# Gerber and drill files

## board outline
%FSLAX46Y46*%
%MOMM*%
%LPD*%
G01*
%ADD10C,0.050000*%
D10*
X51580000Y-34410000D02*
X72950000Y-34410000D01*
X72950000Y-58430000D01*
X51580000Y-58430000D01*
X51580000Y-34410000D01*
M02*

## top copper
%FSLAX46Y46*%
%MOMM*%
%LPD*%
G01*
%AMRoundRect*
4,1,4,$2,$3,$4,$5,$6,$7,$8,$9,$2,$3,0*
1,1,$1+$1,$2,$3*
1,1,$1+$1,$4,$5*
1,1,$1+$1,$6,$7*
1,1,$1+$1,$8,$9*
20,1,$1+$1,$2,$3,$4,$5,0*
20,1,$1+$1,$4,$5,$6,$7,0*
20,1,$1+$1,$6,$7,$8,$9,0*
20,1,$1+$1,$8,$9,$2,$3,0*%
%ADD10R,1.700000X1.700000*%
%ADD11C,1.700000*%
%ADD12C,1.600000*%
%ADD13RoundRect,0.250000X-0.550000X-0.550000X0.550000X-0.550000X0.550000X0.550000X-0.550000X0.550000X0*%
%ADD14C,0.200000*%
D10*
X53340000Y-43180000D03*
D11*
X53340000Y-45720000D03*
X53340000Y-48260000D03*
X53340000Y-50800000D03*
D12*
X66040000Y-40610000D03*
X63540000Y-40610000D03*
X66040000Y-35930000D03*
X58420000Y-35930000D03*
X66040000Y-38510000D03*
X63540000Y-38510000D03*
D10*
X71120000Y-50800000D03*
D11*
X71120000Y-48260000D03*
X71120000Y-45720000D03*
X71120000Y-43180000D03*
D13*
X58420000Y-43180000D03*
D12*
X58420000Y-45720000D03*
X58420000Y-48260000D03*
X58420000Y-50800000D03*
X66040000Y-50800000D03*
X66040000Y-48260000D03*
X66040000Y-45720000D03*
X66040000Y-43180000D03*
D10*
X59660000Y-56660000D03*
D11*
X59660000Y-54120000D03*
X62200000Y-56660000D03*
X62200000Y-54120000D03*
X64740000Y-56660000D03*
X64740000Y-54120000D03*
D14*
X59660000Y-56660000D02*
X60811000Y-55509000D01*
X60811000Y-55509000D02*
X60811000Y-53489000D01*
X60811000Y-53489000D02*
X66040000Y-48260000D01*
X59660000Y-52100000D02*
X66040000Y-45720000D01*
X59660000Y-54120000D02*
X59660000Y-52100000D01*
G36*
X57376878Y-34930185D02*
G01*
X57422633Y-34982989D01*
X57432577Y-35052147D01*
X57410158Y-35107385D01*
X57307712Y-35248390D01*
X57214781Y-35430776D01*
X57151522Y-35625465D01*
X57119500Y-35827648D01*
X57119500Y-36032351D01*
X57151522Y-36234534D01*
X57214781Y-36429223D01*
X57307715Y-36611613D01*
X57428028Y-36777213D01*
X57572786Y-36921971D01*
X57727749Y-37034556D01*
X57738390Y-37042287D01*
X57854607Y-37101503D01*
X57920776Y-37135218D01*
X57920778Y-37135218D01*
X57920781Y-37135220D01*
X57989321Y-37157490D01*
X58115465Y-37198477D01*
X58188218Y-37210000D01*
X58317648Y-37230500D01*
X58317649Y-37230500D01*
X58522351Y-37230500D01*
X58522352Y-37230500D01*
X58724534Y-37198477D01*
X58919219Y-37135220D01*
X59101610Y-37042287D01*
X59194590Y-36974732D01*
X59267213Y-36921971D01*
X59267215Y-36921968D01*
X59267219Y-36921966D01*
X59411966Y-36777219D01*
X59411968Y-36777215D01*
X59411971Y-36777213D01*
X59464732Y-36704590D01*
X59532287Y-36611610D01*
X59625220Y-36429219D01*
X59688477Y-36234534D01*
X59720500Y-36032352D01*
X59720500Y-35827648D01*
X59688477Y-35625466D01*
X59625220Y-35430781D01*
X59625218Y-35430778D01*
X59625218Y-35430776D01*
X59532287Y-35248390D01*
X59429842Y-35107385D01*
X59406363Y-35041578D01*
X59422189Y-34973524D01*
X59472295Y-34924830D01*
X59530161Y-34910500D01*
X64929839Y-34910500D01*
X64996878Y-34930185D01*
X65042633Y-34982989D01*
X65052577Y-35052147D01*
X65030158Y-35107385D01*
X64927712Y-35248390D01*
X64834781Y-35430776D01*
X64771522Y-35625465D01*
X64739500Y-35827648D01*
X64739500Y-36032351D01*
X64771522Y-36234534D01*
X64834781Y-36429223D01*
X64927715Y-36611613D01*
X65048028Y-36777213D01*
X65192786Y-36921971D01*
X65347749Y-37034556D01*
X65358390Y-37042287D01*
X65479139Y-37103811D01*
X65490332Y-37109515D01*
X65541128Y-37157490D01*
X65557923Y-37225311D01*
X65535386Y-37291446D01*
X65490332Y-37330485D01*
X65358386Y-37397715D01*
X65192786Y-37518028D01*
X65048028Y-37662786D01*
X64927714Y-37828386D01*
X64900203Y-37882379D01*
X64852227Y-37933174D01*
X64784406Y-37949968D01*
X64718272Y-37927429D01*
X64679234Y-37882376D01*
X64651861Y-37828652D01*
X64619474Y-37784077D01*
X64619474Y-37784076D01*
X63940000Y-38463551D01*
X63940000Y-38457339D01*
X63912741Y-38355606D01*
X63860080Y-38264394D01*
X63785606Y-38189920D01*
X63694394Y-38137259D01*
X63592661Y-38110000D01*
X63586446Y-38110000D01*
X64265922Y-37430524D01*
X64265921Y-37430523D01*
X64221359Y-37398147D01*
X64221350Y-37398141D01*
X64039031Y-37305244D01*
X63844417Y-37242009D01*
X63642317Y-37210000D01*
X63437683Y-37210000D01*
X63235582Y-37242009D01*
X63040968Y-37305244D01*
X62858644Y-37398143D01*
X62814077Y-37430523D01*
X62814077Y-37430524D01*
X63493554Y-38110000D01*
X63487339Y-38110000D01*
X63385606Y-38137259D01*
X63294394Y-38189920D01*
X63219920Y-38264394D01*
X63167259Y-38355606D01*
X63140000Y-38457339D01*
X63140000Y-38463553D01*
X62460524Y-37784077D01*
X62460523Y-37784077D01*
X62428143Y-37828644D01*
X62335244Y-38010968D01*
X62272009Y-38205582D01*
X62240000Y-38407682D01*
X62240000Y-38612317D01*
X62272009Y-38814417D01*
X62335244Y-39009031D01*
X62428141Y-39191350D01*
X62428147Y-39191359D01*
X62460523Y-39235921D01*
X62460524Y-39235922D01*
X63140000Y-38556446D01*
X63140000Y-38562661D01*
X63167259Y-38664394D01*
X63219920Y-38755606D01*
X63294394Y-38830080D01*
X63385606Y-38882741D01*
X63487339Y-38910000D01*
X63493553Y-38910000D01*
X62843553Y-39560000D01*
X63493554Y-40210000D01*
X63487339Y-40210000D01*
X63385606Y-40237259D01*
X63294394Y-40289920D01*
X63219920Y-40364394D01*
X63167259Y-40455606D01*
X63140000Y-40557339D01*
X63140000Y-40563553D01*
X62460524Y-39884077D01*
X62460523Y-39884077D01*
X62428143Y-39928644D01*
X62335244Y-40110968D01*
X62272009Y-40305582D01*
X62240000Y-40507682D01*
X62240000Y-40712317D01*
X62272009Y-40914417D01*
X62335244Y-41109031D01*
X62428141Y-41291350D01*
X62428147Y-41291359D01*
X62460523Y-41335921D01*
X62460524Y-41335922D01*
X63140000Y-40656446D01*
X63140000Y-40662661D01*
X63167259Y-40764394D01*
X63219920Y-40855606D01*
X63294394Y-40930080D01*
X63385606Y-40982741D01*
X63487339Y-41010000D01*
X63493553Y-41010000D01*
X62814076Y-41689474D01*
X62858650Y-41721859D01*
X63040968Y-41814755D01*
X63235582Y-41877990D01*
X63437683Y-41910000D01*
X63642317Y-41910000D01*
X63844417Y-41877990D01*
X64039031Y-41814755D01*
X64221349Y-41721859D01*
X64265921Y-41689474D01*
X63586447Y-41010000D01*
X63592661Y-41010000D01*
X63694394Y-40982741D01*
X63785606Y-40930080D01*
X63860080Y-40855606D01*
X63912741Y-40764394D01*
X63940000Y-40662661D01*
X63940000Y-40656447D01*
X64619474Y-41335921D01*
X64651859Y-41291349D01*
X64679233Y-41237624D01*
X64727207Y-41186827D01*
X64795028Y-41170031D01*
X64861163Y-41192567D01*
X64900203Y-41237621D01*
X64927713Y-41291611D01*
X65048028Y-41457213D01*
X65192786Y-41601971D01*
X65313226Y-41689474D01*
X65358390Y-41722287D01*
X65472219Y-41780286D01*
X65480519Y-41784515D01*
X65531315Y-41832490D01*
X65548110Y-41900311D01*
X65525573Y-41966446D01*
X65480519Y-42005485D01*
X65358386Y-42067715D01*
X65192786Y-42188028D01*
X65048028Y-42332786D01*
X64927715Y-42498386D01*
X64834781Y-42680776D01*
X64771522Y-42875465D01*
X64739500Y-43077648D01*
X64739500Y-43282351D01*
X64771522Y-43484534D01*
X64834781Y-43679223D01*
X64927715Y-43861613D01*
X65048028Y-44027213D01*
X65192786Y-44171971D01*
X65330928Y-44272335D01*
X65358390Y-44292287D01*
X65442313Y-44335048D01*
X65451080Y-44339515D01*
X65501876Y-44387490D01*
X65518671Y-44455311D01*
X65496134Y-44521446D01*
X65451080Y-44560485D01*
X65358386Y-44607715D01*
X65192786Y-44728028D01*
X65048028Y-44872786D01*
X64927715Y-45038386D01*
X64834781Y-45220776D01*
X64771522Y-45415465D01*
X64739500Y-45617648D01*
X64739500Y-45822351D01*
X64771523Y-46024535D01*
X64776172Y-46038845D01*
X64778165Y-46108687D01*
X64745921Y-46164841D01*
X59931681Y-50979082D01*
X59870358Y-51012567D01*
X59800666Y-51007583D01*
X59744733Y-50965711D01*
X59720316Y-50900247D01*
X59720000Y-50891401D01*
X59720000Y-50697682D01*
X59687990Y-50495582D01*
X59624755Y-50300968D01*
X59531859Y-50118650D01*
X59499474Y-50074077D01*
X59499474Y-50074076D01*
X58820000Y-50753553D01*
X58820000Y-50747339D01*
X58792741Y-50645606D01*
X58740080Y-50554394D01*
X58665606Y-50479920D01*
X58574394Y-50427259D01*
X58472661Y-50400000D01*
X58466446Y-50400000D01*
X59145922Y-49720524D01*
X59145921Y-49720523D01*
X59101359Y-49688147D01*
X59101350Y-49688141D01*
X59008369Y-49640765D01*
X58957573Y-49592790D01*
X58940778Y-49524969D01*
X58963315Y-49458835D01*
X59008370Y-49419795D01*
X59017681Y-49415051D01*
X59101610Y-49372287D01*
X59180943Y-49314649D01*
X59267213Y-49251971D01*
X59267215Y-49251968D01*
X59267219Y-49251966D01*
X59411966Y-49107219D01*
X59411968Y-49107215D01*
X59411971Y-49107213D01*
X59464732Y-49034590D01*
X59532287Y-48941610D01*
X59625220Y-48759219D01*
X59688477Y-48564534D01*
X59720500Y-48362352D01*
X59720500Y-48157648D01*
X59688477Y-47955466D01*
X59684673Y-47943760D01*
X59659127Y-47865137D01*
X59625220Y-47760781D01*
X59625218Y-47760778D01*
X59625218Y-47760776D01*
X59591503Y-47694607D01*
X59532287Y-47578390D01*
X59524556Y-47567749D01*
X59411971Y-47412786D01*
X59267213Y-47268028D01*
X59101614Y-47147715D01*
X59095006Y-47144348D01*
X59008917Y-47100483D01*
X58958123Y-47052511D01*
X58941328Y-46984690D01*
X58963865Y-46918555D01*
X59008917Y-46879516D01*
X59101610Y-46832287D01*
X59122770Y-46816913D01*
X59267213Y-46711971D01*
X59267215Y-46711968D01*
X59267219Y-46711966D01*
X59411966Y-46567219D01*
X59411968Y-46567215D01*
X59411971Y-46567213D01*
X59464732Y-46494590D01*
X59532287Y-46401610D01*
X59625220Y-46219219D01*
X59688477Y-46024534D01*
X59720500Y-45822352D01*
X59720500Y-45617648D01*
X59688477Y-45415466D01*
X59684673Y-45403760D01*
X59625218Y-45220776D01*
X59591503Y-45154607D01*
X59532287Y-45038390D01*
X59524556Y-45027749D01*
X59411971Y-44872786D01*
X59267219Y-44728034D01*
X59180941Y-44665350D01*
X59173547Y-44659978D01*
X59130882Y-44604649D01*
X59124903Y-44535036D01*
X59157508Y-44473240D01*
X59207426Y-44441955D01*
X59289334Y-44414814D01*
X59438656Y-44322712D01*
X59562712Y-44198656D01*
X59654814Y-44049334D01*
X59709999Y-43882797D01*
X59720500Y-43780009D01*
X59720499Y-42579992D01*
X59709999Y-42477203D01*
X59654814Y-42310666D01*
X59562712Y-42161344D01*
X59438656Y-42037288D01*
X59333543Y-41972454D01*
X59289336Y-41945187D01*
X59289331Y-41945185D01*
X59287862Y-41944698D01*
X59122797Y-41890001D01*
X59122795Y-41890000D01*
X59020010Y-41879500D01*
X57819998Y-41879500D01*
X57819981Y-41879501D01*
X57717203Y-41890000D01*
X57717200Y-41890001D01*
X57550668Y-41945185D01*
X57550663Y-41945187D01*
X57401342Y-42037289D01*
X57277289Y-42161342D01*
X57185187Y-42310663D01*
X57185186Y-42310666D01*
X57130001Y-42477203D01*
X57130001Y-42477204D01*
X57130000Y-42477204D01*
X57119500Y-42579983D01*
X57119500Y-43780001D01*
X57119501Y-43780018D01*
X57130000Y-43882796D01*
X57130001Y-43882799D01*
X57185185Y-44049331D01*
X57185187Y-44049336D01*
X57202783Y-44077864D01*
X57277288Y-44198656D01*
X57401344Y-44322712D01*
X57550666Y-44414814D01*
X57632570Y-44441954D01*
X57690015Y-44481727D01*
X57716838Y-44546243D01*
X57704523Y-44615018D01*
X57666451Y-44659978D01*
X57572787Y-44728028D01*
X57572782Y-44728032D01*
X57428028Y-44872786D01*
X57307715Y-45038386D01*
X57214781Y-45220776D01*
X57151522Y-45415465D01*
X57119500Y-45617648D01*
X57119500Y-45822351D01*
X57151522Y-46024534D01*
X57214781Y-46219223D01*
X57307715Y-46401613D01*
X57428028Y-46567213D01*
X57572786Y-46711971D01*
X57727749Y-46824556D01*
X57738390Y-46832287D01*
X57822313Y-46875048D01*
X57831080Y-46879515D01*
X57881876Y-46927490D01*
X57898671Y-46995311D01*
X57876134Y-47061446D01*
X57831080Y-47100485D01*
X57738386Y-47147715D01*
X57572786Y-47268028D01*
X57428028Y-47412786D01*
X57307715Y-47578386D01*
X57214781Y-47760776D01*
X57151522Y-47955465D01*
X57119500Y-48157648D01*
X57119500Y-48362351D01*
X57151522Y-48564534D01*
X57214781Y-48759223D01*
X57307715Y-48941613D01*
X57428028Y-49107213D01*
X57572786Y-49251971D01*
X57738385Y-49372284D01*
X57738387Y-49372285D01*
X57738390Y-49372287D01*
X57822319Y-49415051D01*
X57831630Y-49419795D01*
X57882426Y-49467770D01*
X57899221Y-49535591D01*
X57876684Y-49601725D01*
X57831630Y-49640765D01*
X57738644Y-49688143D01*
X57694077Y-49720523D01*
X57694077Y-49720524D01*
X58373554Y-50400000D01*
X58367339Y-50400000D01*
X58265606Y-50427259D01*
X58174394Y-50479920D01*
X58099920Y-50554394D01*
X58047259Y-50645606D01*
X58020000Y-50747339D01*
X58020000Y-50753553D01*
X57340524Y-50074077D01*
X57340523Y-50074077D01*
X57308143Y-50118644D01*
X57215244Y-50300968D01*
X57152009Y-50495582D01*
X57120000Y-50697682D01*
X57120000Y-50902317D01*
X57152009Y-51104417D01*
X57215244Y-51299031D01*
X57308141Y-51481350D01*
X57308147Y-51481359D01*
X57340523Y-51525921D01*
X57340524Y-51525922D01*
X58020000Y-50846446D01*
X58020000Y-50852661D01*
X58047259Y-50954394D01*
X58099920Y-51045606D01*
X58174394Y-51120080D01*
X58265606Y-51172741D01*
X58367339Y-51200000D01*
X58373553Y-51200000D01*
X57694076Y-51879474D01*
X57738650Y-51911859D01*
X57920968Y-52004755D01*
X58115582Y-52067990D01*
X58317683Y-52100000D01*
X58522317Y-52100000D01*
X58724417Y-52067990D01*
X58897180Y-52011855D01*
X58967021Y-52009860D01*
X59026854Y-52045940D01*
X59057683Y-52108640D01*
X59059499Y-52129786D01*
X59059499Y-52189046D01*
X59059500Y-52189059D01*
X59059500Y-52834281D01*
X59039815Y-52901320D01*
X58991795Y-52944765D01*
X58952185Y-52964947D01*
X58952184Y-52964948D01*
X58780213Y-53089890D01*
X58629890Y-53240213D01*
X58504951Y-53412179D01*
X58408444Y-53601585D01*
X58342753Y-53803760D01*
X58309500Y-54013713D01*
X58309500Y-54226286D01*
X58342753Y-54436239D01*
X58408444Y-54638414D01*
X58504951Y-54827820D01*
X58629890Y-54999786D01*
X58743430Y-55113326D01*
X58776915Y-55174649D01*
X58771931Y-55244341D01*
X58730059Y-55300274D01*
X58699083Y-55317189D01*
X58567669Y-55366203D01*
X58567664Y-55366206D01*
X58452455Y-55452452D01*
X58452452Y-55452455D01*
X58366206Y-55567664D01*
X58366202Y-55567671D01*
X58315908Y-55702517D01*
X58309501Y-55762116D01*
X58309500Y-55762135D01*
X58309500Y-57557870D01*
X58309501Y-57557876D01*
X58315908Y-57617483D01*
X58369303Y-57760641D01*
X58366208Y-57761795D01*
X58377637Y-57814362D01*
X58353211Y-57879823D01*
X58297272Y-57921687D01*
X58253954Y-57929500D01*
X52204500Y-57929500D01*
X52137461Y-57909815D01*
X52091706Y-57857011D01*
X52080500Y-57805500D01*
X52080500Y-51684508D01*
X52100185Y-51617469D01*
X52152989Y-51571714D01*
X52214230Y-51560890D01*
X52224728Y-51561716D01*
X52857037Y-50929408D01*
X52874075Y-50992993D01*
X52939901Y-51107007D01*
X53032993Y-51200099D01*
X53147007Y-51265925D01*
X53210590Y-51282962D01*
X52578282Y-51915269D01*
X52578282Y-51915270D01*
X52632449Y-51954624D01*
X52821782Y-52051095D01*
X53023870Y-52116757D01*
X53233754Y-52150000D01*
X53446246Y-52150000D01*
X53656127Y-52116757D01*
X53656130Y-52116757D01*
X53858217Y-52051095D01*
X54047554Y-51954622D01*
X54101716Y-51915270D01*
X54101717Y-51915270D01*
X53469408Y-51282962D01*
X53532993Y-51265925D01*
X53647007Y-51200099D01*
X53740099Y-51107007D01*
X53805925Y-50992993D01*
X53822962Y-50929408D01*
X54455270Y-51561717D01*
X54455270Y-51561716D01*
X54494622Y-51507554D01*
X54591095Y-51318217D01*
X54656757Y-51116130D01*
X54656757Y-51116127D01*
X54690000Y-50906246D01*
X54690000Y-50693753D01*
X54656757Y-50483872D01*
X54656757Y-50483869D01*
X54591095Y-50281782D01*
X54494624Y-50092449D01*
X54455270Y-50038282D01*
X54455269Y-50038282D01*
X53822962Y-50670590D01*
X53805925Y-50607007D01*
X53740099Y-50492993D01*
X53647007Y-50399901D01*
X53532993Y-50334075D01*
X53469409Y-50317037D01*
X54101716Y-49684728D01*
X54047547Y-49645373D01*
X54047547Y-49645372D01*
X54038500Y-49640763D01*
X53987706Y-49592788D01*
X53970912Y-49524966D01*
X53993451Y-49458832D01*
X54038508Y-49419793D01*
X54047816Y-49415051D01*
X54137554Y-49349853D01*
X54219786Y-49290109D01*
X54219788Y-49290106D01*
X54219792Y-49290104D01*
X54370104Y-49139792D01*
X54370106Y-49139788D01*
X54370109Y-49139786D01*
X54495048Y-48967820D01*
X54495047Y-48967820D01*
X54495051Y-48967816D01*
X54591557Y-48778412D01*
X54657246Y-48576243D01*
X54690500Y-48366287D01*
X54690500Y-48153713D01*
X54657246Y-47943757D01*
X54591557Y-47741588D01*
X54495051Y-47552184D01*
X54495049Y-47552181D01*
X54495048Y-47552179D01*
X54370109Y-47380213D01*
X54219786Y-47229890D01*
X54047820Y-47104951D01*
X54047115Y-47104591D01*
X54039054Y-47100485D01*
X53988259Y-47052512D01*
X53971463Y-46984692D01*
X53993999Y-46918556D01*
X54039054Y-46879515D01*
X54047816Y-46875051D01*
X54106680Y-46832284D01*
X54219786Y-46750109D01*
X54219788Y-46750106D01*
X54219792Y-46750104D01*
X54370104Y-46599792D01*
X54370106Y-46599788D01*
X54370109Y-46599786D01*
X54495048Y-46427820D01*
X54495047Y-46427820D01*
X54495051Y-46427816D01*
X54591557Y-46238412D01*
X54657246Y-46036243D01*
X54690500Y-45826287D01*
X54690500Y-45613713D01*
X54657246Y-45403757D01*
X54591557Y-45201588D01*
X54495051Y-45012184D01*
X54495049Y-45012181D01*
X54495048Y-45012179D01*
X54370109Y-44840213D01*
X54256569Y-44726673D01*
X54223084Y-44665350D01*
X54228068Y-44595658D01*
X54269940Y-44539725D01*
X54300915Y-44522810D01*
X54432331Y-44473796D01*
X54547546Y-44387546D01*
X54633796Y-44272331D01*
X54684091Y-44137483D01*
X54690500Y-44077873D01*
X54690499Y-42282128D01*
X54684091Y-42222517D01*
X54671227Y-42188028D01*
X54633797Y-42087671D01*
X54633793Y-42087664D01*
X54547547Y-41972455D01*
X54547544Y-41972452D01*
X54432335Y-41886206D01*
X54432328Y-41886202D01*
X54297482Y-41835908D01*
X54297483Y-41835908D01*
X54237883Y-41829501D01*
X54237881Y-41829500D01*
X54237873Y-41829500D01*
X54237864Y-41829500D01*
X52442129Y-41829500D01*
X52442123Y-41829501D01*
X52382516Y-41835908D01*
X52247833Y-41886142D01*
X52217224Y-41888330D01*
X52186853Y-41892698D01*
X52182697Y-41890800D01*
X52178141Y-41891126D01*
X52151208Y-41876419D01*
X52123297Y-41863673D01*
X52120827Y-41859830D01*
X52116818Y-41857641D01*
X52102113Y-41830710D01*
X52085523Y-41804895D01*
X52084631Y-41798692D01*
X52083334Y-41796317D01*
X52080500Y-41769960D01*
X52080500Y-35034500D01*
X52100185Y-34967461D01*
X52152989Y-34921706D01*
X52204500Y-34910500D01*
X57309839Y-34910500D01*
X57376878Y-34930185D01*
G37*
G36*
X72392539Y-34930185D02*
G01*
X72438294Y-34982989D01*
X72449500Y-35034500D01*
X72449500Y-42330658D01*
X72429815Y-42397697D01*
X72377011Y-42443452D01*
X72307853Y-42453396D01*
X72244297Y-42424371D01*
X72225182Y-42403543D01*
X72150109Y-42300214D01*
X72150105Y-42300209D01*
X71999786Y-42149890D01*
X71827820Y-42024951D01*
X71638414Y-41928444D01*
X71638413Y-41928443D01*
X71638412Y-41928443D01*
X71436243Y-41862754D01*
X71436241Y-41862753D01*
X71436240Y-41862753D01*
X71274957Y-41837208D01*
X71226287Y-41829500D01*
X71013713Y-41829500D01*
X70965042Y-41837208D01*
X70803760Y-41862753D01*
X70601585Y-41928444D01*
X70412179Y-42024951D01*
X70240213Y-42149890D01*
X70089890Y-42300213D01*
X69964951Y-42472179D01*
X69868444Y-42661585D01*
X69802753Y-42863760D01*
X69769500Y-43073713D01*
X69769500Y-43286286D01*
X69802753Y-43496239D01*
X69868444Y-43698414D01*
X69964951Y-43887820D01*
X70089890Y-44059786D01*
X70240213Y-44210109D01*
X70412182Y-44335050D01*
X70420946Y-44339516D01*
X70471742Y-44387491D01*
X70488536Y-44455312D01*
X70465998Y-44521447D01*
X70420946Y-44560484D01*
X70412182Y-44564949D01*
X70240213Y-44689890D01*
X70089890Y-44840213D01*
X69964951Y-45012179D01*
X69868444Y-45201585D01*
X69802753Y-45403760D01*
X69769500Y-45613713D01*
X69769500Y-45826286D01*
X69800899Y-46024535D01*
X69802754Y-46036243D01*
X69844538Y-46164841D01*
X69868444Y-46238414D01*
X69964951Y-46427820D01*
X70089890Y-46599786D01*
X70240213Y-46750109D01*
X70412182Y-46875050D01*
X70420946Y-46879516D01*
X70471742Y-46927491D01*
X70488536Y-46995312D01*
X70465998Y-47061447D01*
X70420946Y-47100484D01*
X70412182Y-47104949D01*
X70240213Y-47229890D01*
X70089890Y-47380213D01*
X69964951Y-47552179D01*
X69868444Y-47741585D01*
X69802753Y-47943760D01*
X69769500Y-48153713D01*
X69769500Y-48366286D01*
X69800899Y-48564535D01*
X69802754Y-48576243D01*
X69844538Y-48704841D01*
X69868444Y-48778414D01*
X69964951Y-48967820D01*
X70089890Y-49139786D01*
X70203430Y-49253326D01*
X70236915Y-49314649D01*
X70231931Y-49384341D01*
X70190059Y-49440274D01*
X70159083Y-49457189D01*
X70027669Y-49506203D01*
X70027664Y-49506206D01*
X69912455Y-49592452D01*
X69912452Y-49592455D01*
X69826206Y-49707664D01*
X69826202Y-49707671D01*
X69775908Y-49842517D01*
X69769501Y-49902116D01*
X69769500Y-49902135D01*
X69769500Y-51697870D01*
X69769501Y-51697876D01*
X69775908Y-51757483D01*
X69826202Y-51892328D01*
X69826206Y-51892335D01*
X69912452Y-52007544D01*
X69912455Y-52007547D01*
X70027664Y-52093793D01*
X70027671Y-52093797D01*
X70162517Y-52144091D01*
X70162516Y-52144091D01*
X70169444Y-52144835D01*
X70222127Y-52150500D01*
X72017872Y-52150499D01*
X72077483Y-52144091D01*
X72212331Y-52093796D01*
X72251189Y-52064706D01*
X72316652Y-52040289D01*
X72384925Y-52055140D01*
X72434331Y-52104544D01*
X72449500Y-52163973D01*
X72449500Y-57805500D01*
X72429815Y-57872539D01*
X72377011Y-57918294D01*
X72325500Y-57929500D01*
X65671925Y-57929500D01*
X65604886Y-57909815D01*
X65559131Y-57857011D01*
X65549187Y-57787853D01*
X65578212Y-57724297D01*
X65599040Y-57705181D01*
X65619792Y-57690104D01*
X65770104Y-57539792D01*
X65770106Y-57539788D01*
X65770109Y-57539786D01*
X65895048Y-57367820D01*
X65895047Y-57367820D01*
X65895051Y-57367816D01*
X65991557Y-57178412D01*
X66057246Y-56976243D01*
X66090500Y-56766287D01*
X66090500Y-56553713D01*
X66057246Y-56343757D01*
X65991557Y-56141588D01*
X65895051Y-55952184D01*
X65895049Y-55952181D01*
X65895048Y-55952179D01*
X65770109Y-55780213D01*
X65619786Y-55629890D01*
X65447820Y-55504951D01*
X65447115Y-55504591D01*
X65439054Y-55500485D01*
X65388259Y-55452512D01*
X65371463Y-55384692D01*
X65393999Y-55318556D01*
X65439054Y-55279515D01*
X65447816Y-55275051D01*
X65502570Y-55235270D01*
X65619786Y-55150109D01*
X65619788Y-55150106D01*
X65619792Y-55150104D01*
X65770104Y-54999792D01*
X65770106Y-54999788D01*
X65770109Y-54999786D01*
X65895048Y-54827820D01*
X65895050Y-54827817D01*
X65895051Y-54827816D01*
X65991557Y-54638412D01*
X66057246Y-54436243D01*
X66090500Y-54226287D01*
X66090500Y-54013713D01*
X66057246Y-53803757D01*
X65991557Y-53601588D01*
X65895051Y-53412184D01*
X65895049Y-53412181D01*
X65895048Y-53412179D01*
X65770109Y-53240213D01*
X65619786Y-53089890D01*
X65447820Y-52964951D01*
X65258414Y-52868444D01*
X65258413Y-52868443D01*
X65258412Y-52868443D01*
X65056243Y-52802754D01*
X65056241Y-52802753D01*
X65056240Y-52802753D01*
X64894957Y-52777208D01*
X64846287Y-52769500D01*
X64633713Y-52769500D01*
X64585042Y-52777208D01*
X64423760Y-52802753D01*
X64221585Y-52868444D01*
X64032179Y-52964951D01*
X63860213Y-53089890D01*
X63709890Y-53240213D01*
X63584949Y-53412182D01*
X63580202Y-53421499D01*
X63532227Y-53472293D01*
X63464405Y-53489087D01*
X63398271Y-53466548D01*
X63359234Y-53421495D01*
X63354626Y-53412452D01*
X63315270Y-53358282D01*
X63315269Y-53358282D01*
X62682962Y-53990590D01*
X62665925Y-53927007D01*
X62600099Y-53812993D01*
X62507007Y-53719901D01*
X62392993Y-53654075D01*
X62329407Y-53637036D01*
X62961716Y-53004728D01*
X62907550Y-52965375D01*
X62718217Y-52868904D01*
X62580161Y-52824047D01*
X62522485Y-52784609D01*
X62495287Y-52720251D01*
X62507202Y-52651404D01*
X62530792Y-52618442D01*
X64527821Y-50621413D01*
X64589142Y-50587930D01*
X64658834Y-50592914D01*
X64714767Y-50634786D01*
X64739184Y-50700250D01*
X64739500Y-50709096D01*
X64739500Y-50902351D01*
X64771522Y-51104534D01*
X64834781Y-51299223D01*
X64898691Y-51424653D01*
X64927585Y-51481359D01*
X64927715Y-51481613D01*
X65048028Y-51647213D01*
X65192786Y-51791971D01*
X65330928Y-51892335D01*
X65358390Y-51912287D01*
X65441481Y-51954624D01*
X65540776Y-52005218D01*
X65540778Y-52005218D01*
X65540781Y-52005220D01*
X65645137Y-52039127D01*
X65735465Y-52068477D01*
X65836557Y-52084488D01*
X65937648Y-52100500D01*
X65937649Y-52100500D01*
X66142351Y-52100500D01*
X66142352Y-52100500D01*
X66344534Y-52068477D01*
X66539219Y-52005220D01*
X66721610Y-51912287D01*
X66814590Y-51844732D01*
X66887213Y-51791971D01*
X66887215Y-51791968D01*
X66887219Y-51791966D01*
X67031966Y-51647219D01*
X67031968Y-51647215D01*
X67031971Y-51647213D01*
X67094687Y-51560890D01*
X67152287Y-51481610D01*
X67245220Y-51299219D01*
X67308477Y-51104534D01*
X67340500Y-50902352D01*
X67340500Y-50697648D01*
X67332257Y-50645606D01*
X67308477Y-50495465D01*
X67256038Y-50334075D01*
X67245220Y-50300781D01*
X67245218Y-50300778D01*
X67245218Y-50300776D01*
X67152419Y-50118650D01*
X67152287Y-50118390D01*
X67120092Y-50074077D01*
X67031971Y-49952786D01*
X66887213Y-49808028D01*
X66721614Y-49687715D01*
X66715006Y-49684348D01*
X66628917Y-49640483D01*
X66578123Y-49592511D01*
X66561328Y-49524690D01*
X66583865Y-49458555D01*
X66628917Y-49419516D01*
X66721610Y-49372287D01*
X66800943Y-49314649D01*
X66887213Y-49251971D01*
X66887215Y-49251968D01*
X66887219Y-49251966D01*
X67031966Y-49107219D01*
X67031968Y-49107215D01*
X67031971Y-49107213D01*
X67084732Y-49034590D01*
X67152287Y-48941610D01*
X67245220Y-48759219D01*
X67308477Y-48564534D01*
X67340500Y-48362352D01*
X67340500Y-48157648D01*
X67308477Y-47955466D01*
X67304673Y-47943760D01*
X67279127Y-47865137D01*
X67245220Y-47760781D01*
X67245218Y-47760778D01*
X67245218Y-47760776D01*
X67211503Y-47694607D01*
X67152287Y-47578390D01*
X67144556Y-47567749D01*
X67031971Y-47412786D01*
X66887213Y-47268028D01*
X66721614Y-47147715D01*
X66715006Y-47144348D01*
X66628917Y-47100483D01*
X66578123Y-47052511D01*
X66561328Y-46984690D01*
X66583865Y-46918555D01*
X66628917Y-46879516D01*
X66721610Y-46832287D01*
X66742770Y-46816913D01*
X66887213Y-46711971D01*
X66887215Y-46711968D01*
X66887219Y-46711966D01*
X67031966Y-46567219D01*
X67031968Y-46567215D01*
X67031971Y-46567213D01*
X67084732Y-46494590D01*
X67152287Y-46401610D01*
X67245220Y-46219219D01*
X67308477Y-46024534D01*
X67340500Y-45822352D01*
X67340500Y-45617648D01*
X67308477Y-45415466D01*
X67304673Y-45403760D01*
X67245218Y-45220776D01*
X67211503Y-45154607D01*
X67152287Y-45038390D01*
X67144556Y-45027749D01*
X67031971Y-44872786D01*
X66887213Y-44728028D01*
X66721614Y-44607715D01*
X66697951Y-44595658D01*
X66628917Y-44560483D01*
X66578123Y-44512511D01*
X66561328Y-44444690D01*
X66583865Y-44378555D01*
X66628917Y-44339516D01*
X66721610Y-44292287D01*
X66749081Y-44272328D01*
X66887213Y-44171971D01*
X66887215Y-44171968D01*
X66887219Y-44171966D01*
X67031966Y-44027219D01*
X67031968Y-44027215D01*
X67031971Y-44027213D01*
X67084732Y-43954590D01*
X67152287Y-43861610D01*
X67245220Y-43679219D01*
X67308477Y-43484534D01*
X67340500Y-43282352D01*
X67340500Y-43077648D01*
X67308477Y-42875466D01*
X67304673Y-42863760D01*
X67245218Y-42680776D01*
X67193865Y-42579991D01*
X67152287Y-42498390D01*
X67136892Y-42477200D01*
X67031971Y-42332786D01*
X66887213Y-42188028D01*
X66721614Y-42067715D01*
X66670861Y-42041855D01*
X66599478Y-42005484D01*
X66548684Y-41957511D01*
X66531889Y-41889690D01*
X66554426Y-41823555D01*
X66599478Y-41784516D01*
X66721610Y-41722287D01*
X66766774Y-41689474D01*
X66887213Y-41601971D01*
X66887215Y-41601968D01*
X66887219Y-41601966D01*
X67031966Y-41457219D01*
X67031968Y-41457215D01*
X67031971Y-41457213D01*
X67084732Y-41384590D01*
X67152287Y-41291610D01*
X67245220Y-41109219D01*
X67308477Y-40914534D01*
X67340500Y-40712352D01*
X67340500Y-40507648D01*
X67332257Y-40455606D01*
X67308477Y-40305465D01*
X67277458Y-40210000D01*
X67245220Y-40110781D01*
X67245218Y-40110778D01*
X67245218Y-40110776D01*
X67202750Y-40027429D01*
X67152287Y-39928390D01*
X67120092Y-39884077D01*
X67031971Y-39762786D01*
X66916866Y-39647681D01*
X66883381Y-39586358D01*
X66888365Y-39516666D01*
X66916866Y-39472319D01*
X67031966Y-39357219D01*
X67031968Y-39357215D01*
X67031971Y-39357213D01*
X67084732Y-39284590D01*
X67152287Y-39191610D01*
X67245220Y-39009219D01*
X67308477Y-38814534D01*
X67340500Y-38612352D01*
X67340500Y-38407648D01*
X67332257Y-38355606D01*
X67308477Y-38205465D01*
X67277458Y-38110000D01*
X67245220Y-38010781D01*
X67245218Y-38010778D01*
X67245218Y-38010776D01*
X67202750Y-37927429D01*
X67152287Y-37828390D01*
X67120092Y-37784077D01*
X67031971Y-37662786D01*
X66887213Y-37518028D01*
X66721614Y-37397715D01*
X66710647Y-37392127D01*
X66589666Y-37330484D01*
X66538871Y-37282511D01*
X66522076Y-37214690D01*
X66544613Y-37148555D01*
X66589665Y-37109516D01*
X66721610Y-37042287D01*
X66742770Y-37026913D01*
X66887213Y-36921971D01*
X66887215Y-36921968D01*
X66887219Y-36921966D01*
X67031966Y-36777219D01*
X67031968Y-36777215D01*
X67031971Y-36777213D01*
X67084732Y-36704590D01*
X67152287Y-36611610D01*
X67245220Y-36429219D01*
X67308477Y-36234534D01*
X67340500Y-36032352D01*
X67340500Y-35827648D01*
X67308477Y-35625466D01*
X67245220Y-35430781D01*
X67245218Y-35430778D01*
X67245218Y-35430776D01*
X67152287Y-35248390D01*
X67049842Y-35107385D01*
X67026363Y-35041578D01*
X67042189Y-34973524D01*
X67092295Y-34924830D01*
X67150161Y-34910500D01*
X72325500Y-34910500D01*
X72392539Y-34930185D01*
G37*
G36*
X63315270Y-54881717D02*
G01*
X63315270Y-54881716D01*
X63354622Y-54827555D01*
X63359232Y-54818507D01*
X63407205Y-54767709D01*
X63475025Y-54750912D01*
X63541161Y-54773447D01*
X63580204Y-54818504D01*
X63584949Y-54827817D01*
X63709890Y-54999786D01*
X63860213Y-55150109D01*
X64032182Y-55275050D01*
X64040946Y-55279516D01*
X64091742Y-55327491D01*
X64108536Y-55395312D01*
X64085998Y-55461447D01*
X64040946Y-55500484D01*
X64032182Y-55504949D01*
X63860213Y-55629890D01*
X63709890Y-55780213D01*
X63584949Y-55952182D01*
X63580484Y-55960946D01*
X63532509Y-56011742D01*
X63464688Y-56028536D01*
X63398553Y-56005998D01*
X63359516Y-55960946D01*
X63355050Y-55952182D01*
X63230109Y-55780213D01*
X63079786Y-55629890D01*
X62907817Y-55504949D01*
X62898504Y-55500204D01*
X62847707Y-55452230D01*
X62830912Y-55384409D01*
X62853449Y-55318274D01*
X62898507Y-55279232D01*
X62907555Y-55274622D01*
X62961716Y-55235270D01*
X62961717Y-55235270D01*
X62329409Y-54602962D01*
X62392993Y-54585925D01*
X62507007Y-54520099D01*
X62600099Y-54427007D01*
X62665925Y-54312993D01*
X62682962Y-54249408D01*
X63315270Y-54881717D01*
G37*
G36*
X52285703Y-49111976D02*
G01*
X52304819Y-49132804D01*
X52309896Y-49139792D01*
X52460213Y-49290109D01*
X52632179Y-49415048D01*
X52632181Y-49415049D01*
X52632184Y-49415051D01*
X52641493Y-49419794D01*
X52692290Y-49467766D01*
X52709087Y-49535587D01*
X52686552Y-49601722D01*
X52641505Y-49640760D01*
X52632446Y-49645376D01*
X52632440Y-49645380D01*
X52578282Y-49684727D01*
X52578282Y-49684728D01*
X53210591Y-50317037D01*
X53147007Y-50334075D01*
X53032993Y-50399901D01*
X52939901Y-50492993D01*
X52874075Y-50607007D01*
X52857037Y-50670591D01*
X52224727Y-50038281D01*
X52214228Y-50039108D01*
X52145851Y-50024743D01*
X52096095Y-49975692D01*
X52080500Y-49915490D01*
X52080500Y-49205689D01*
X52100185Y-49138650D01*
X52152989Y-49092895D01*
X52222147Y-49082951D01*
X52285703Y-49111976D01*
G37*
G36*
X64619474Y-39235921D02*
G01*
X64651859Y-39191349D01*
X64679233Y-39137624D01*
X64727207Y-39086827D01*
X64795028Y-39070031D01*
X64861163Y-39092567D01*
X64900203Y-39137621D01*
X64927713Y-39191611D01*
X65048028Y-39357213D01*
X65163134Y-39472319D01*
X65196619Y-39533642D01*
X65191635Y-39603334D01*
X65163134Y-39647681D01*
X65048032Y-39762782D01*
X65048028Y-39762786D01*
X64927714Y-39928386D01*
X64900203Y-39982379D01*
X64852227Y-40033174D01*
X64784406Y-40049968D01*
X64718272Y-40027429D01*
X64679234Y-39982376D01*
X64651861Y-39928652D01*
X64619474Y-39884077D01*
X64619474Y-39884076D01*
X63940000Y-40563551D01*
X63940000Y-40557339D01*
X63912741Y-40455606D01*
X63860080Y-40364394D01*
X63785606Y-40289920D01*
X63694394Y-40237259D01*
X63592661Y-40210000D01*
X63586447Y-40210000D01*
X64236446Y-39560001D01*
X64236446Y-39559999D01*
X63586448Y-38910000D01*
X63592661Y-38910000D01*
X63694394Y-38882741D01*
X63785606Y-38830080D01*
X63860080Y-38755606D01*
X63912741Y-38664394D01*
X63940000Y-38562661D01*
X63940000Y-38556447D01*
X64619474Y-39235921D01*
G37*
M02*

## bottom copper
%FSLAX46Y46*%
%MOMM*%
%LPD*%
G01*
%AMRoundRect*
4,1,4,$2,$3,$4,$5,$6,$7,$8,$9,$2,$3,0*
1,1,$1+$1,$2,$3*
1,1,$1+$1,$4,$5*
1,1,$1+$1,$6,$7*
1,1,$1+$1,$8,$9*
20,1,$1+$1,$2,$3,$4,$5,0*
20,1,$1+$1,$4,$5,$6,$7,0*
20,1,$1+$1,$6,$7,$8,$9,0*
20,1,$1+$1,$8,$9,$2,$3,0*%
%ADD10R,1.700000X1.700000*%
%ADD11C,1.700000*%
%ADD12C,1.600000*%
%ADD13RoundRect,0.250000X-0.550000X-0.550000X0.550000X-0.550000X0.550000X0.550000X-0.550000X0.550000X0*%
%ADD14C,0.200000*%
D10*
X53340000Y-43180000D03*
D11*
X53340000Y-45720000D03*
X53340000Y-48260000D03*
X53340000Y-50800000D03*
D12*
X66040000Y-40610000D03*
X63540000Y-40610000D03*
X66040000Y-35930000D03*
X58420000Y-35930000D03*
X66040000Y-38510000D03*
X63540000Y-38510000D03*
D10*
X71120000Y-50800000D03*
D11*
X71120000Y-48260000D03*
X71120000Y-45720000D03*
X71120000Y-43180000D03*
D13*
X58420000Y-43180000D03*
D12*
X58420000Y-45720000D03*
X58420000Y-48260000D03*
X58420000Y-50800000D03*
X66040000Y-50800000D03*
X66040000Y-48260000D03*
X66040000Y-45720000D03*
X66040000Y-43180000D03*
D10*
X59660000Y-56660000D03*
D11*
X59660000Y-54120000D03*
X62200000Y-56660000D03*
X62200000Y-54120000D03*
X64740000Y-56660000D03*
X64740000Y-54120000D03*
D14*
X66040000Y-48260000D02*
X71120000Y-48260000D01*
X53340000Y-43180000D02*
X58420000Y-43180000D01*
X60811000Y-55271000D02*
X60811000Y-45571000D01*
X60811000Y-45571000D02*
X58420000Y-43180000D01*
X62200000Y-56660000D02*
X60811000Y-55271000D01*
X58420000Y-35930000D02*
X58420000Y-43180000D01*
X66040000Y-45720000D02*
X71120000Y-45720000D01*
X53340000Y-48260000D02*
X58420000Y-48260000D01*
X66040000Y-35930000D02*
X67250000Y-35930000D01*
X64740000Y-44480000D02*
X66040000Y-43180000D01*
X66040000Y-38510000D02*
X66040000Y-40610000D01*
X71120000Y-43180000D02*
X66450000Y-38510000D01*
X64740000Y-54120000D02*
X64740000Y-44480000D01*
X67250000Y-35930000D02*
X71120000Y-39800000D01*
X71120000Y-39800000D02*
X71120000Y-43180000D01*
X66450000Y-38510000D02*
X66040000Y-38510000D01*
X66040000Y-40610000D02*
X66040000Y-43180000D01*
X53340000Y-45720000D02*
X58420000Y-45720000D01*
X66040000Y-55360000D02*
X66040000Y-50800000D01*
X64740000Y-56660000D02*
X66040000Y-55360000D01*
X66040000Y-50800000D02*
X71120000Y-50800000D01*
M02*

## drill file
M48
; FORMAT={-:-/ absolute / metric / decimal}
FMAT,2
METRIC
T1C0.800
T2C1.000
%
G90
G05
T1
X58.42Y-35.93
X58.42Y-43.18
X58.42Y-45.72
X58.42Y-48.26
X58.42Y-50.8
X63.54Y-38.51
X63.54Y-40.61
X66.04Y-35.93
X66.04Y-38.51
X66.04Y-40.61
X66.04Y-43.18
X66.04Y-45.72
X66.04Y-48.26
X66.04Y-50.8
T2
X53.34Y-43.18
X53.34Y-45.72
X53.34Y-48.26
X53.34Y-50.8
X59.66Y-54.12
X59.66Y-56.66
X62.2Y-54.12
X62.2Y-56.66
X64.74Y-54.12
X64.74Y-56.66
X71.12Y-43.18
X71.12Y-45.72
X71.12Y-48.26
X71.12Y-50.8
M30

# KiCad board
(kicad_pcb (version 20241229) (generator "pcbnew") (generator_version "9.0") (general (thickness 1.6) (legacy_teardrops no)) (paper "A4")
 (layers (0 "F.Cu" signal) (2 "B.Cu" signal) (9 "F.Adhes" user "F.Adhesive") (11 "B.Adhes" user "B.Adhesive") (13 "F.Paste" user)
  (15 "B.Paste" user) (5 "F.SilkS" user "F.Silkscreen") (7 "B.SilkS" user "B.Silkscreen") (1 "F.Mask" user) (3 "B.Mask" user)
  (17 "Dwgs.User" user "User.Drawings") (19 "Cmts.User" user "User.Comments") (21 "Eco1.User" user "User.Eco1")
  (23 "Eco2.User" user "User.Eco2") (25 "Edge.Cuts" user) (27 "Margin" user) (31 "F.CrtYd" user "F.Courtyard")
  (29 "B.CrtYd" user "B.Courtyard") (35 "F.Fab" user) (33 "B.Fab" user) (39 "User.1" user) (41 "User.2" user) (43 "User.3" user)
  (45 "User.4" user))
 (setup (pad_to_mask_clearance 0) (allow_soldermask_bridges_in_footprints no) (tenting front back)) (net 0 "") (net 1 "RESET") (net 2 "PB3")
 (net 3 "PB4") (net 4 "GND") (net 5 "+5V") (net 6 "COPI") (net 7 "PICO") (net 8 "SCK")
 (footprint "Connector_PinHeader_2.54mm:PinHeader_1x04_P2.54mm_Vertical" (layer "F.Cu") (at 53.34 43.18)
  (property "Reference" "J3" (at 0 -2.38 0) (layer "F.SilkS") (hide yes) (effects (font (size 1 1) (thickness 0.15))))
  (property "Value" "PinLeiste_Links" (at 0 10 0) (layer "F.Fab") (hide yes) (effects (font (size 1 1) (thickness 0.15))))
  (pad "1" thru_hole rect (at 0 0) (size 1.7 1.7) (drill 1) (layers "*.Cu" "*.Mask") (remove_unused_layers no) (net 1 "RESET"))
  (pad "2" thru_hole circle (at 0 2.54) (size 1.7 1.7) (drill 1) (layers "*.Cu" "*.Mask") (remove_unused_layers no) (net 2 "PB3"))
  (pad "3" thru_hole circle (at 0 5.08) (size 1.7 1.7) (drill 1) (layers "*.Cu" "*.Mask") (remove_unused_layers no) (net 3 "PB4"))
  (pad "4" thru_hole circle (at 0 7.62) (size 1.7 1.7) (drill 1) (layers "*.Cu" "*.Mask") (remove_unused_layers no) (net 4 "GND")))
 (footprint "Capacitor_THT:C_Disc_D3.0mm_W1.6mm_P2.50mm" (layer "F.Cu") (at 66.04 40.61 180)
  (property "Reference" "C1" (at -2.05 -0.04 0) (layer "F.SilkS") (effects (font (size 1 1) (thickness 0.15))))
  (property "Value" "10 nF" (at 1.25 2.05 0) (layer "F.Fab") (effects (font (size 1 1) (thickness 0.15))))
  (pad "1" thru_hole circle (at 0 0 180) (size 1.6 1.6) (drill 0.8) (layers "*.Cu" "*.Mask") (remove_unused_layers no) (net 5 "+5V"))
  (pad "2" thru_hole circle (at 2.5 0 180) (size 1.6 1.6) (drill 0.8) (layers "*.Cu" "*.Mask") (remove_unused_layers no) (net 4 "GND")))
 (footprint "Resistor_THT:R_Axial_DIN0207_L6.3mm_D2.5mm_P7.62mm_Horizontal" (layer "F.Cu") (at 66.04 35.93 180)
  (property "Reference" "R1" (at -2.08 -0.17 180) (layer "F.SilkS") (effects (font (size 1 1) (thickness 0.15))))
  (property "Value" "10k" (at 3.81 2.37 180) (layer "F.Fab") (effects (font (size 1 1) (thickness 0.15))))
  (pad "1" thru_hole circle (at 0 0 180) (size 1.6 1.6) (drill 0.8) (layers "*.Cu" "*.Mask") (remove_unused_layers no) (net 5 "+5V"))
  (pad "2" thru_hole circle (at 7.62 0 180) (size 1.6 1.6) (drill 0.8) (layers "*.Cu" "*.Mask") (remove_unused_layers no) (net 1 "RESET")))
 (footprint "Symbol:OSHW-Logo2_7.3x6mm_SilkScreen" (layer "F.Cu") (at 55.14 38.13)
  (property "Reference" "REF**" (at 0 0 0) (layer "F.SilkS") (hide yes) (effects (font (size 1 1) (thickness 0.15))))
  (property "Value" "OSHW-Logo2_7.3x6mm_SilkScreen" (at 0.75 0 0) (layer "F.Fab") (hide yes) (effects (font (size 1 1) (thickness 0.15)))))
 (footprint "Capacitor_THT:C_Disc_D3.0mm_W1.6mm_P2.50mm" (layer "F.Cu") (at 66.04 38.51 180)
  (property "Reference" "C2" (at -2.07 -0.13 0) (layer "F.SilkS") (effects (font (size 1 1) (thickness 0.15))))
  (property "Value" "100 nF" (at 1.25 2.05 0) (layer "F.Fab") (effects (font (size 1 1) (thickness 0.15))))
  (pad "1" thru_hole circle (at 0 0 180) (size 1.6 1.6) (drill 0.8) (layers "*.Cu" "*.Mask") (remove_unused_layers no) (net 5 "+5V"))
  (pad "2" thru_hole circle (at 2.5 0 180) (size 1.6 1.6) (drill 0.8) (layers "*.Cu" "*.Mask") (remove_unused_layers no) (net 4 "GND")))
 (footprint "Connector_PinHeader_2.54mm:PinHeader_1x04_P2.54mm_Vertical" (layer "F.Cu") (at 71.12 50.8 180)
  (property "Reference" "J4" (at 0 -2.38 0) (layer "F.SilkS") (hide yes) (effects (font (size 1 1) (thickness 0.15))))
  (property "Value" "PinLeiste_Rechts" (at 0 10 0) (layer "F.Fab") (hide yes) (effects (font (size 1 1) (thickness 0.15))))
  (pad "1" thru_hole rect (at 0 0 180) (size 1.7 1.7) (drill 1) (layers "*.Cu" "*.Mask") (remove_unused_layers no) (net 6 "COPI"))
  (pad "2" thru_hole circle (at 0 2.54 180) (size 1.7 1.7) (drill 1) (layers "*.Cu" "*.Mask") (remove_unused_layers no) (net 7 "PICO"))
  (pad "3" thru_hole circle (at 0 5.08 180) (size 1.7 1.7) (drill 1) (layers "*.Cu" "*.Mask") (remove_unused_layers no) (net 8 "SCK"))
  (pad "4" thru_hole circle (at 0 7.62 180) (size 1.7 1.7) (drill 1) (layers "*.Cu" "*.Mask") (remove_unused_layers no) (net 5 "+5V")))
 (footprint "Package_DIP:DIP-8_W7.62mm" (layer "F.Cu") (at 58.42 43.18)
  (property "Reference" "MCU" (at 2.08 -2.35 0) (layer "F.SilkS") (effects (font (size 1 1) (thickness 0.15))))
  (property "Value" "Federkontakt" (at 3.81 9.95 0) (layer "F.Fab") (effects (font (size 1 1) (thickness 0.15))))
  (pad "1" thru_hole roundrect (at 0 0) (size 1.6 1.6) (drill 0.8) (layers "*.Cu" "*.Mask") (remove_unused_layers no)
   (roundrect_rratio 0.15625) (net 1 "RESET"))
  (pad "2" thru_hole circle (at 0 2.54) (size 1.6 1.6) (drill 0.8) (layers "*.Cu" "*.Mask") (remove_unused_layers no) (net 2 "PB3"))
  (pad "3" thru_hole circle (at 0 5.08) (size 1.6 1.6) (drill 0.8) (layers "*.Cu" "*.Mask") (remove_unused_layers no) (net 3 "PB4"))
  (pad "4" thru_hole circle (at 0 7.62) (size 1.6 1.6) (drill 0.8) (layers "*.Cu" "*.Mask") (remove_unused_layers no) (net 4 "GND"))
  (pad "5" thru_hole circle (at 7.62 7.62) (size 1.6 1.6) (drill 0.8) (layers "*.Cu" "*.Mask") (remove_unused_layers no) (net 6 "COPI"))
  (pad "6" thru_hole circle (at 7.62 5.08) (size 1.6 1.6) (drill 0.8) (layers "*.Cu" "*.Mask") (remove_unused_layers no) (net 7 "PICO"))
  (pad "7" thru_hole circle (at 7.62 2.54) (size 1.6 1.6) (drill 0.8) (layers "*.Cu" "*.Mask") (remove_unused_layers no) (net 8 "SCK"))
  (pad "8" thru_hole circle (at 7.62 0) (size 1.6 1.6) (drill 0.8) (layers "*.Cu" "*.Mask") (remove_unused_layers no) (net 5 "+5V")))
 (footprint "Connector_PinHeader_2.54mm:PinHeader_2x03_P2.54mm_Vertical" (layer "F.Cu") (at 59.66 56.66 90)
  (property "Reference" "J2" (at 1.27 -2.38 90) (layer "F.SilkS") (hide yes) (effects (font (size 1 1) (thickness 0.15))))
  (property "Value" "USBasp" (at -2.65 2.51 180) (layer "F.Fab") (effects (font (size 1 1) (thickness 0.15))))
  (pad "1" thru_hole rect (at 0 0 90) (size 1.7 1.7) (drill 1) (layers "*.Cu" "*.Mask") (remove_unused_layers no) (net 7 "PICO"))
  (pad "2" thru_hole circle (at 2.54 0 90) (size 1.7 1.7) (drill 1) (layers "*.Cu" "*.Mask") (remove_unused_layers no) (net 8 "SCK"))
  (pad "3" thru_hole circle (at 0 2.54 90) (size 1.7 1.7) (drill 1) (layers "*.Cu" "*.Mask") (remove_unused_layers no) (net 1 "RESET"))
  (pad "4" thru_hole circle (at 2.54 2.54 90) (size 1.7 1.7) (drill 1) (layers "*.Cu" "*.Mask") (remove_unused_layers no) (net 4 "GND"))
  (pad "5" thru_hole circle (at 0 5.08 90) (size 1.7 1.7) (drill 1) (layers "*.Cu" "*.Mask") (remove_unused_layers no) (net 6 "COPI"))
  (pad "6" thru_hole circle (at 2.54 5.08 90) (size 1.7 1.7) (drill 1) (layers "*.Cu" "*.Mask") (remove_unused_layers no) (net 5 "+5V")))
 (gr_rect (start 51.58 34.41) (end 72.95 58.43) (stroke (width 0.05) (type default)) (fill no) (layer "Edge.Cuts"))
 (segment (start 59.66 56.66) (end 60.811 55.509) (width 0.2) (layer "F.Cu") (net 7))
 (segment (start 60.811 55.509) (end 60.811 53.489) (width 0.2) (layer "F.Cu") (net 7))
 (segment (start 60.811 53.489) (end 66.04 48.26) (width 0.2) (layer "F.Cu") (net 7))
 (segment (start 66.04 48.26) (end 71.12 48.26) (width 0.2) (layer "B.Cu") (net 7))
 (segment (start 53.34 43.18) (end 58.42 43.18) (width 0.2) (layer "B.Cu") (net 1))
 (segment (start 60.811 55.271) (end 60.811 45.571) (width 0.2) (layer "B.Cu") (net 1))
 (segment (start 60.811 45.571) (end 58.42 43.18) (width 0.2) (layer "B.Cu") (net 1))
 (segment (start 62.2 56.66) (end 60.811 55.271) (width 0.2) (layer "B.Cu") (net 1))
 (segment (start 58.42 35.93) (end 58.42 43.18) (width 0.2) (layer "B.Cu") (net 1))
 (segment (start 59.66 52.1) (end 66.04 45.72) (width 0.2) (layer "F.Cu") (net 8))
 (segment (start 59.66 54.12) (end 59.66 52.1) (width 0.2) (layer "F.Cu") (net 8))
 (segment (start 66.04 45.72) (end 71.12 45.72) (width 0.2) (layer "B.Cu") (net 8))
 (segment (start 53.34 48.26) (end 58.42 48.26) (width 0.2) (layer "B.Cu") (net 3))
 (segment (start 66.04 35.93) (end 67.25 35.93) (width 0.2) (layer "B.Cu") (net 5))
 (segment (start 64.74 44.48) (end 66.04 43.18) (width 0.2) (layer "B.Cu") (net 5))
 (segment (start 66.04 38.51) (end 66.04 40.61) (width 0.2) (layer "B.Cu") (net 5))
 (segment (start 71.12 43.18) (end 66.45 38.51) (width 0.2) (layer "B.Cu") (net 5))
 (segment (start 64.74 54.12) (end 64.74 44.48) (width 0.2) (layer "B.Cu") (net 5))
 (segment (start 67.25 35.93) (end 71.12 39.8) (width 0.2) (layer "B.Cu") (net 5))
 (segment (start 71.12 39.8) (end 71.12 43.18) (width 0.2) (layer "B.Cu") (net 5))
 (segment (start 66.45 38.51) (end 66.04 38.51) (width 0.2) (layer "B.Cu") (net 5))
 (segment (start 66.04 40.61) (end 66.04 43.18) (width 0.2) (layer "B.Cu") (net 5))
 (segment (start 53.34 45.72) (end 58.42 45.72) (width 0.2) (layer "B.Cu") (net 2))
 (segment (start 66.04 55.36) (end 66.04 50.8) (width 0.2) (layer "B.Cu") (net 6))
 (segment (start 64.74 56.66) (end 66.04 55.36) (width 0.2) (layer "B.Cu") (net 6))
 (segment (start 66.04 50.8) (end 71.12 50.8) (width 0.2) (layer "B.Cu") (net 6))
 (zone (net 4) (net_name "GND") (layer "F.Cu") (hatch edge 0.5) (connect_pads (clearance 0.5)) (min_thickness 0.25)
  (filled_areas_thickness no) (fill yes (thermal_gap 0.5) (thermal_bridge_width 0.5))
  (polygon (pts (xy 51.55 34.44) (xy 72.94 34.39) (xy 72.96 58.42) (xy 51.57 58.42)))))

